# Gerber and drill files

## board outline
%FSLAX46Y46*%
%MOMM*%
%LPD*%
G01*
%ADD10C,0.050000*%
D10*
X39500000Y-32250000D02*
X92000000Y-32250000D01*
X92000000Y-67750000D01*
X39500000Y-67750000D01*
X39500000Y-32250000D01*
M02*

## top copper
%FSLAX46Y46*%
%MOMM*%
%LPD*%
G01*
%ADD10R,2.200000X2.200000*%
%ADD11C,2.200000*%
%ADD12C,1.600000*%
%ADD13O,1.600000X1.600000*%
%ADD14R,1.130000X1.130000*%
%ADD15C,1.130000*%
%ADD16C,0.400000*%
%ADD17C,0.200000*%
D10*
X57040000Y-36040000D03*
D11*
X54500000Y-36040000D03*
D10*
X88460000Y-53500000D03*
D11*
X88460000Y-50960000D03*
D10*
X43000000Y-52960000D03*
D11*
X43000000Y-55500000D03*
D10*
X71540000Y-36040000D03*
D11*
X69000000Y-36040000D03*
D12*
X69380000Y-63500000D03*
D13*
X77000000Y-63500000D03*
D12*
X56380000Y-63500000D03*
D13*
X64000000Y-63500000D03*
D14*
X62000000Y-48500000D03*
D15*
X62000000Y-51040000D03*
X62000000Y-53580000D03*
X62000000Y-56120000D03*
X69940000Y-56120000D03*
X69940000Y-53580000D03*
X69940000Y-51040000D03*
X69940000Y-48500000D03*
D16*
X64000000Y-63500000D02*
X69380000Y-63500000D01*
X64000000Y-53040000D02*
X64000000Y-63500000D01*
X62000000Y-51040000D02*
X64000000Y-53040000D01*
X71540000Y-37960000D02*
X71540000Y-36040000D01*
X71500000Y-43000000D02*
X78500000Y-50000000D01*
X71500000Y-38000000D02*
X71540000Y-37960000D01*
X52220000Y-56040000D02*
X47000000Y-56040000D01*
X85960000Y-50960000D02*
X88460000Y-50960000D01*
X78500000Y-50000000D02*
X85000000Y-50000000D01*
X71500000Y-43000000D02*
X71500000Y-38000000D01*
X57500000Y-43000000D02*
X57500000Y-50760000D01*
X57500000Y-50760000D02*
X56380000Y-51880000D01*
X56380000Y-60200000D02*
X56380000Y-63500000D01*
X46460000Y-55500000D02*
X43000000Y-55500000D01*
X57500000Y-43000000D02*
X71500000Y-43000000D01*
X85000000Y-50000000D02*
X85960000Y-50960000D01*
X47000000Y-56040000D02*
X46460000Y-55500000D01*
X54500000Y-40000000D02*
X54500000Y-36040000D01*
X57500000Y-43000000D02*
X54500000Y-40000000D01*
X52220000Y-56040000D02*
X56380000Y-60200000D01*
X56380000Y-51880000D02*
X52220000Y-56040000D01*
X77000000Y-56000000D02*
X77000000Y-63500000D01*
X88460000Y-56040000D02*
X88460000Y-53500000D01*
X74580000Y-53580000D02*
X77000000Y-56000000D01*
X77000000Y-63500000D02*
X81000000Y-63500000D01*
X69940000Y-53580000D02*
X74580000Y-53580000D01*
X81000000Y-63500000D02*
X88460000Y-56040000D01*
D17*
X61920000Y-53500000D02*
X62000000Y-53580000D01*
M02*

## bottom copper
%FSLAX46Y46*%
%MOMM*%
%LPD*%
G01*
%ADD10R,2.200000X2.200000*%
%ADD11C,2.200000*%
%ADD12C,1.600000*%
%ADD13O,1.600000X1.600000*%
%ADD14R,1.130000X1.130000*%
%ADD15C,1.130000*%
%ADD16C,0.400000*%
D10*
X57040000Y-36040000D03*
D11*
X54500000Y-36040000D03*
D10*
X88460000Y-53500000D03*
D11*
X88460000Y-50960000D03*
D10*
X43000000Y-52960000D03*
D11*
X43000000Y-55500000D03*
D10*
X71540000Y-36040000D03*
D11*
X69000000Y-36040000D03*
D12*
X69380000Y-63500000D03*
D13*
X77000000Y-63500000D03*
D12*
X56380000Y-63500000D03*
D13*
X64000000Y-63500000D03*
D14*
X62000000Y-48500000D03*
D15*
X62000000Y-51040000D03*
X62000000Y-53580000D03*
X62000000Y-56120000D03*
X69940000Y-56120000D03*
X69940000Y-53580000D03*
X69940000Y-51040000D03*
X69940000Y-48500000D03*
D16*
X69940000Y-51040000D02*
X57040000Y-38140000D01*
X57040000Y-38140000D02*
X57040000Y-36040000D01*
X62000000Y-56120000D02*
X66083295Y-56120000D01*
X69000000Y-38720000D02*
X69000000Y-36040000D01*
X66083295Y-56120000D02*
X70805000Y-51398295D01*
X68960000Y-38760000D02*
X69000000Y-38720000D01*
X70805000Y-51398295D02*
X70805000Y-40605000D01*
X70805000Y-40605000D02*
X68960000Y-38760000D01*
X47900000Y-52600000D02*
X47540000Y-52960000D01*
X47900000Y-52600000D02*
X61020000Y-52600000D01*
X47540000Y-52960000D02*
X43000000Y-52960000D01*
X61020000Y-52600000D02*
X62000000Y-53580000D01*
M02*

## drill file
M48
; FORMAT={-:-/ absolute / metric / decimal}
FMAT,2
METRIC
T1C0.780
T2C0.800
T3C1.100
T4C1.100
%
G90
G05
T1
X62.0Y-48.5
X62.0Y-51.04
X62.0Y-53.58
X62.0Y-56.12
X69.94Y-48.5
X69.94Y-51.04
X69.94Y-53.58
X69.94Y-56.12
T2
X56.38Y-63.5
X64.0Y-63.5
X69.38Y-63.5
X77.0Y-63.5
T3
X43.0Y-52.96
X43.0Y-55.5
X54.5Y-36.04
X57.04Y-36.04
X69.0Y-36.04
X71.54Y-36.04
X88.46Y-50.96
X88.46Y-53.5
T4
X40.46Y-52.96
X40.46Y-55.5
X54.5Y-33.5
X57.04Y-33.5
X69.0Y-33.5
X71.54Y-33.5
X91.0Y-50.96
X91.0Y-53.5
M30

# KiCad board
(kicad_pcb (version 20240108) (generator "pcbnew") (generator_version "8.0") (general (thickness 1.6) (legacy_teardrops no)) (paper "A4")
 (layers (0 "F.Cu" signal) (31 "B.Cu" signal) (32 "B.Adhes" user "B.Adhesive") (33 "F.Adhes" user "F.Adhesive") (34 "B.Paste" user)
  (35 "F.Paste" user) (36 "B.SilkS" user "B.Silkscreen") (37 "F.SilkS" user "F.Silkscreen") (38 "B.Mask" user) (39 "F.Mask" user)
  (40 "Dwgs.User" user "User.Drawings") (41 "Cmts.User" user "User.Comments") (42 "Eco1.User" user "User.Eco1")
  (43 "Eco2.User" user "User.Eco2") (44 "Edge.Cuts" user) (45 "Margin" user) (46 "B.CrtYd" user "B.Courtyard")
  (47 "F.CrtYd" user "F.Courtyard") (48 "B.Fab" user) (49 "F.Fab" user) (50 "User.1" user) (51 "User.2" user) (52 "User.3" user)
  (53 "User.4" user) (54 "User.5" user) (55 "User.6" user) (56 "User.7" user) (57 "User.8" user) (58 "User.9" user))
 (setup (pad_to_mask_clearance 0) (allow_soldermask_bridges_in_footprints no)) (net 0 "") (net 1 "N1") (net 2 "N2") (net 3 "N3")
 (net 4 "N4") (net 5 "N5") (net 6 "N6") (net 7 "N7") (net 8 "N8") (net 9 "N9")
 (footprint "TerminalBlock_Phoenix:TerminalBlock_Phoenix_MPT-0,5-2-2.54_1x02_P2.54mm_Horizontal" (layer "F.Cu") (at 57.04 36.04 180)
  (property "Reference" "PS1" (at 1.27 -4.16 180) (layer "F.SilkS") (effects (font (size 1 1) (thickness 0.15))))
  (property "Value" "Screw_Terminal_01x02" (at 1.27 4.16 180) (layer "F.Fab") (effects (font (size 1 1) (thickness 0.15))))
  (pad "" np_thru_hole circle (at 0 2.54 180) (size 1.1 1.1) (drill 1.1) (layers "*.Cu" "*.Mask"))
  (pad "" np_thru_hole circle (at 2.54 2.54 180) (size 1.1 1.1) (drill 1.1) (layers "*.Cu" "*.Mask"))
  (pad "1" thru_hole rect (at 0 0 180) (size 2.2 2.2) (drill 1.1) (layers "*.Cu" "*.Mask") (remove_unused_layers no) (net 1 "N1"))
  (pad "2" thru_hole circle (at 2.54 0 180) (size 2.2 2.2) (drill 1.1) (layers "*.Cu" "*.Mask") (remove_unused_layers no) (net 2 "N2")))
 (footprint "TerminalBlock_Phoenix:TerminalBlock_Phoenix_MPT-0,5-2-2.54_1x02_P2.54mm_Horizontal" (layer "F.Cu") (at 88.46 53.5 90)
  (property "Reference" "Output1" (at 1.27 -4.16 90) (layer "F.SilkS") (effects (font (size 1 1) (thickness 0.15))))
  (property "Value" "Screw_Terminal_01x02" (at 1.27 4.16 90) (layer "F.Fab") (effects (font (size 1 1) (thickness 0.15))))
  (pad "" np_thru_hole circle (at 0 2.54 90) (size 1.1 1.1) (drill 1.1) (layers "*.Cu" "*.Mask"))
  (pad "" np_thru_hole circle (at 2.54 2.54 90) (size 1.1 1.1) (drill 1.1) (layers "*.Cu" "*.Mask"))
  (pad "1" thru_hole rect (at 0 0 90) (size 2.2 2.2) (drill 1.1) (layers "*.Cu" "*.Mask") (remove_unused_layers no) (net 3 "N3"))
  (pad "2" thru_hole circle (at 2.54 0 90) (size 2.2 2.2) (drill 1.1) (layers "*.Cu" "*.Mask") (remove_unused_layers no) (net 2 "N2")))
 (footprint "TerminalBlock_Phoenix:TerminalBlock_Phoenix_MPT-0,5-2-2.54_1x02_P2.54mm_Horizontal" (layer "F.Cu") (at 43 52.96 -90)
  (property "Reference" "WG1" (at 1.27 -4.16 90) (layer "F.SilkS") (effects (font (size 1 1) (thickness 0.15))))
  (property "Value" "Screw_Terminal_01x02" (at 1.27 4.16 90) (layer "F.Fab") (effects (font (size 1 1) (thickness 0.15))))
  (pad "" np_thru_hole circle (at 0 2.54 270) (size 1.1 1.1) (drill 1.1) (layers "*.Cu" "*.Mask"))
  (pad "" np_thru_hole circle (at 2.54 2.54 270) (size 1.1 1.1) (drill 1.1) (layers "*.Cu" "*.Mask"))
  (pad "1" thru_hole rect (at 0 0 270) (size 2.2 2.2) (drill 1.1) (layers "*.Cu" "*.Mask") (remove_unused_layers no) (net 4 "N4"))
  (pad "2" thru_hole circle (at 2.54 0 270) (size 2.2 2.2) (drill 1.1) (layers "*.Cu" "*.Mask") (remove_unused_layers no) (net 2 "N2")))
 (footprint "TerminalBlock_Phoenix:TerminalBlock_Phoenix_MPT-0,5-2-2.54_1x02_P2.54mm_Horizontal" (layer "F.Cu") (at 71.54 36.04 180)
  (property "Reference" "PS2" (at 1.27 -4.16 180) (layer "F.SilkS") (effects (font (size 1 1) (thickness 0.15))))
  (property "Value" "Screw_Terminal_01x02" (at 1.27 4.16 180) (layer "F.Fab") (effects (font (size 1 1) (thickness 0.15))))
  (pad "" np_thru_hole circle (at 0 2.54 180) (size 1.1 1.1) (drill 1.1) (layers "*.Cu" "*.Mask"))
  (pad "" np_thru_hole circle (at 2.54 2.54 180) (size 1.1 1.1) (drill 1.1) (layers "*.Cu" "*.Mask"))
  (pad "1" thru_hole rect (at 0 0 180) (size 2.2 2.2) (drill 1.1) (layers "*.Cu" "*.Mask") (remove_unused_layers no) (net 2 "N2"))
  (pad "2" thru_hole circle (at 2.54 0 180) (size 2.2 2.2) (drill 1.1) (layers "*.Cu" "*.Mask") (remove_unused_layers no) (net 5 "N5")))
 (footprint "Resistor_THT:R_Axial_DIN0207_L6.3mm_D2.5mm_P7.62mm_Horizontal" (layer "F.Cu") (at 69.38 63.5)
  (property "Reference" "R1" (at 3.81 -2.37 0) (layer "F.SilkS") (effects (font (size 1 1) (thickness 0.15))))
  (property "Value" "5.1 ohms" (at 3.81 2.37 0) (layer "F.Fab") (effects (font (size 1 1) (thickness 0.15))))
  (pad "1" thru_hole circle (at 0 0) (size 1.6 1.6) (drill 0.8) (layers "*.Cu" "*.Mask") (remove_unused_layers no) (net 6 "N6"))
  (pad "2" thru_hole oval (at 7.62 0) (size 1.6 1.6) (drill 0.8) (layers "*.Cu" "*.Mask") (remove_unused_layers no) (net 3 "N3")))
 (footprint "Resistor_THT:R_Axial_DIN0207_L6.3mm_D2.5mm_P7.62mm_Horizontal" (layer "F.Cu") (at 56.38 63.5)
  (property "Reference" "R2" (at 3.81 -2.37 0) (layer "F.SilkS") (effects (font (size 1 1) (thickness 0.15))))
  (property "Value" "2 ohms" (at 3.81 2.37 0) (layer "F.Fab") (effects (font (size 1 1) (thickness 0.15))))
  (pad "1" thru_hole circle (at 0 0) (size 1.6 1.6) (drill 0.8) (layers "*.Cu" "*.Mask") (remove_unused_layers no) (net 2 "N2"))
  (pad "2" thru_hole oval (at 7.62 0) (size 1.6 1.6) (drill 0.8) (layers "*.Cu" "*.Mask") (remove_unused_layers no) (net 6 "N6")))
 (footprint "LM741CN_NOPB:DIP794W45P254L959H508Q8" (layer "F.Cu") (at 65.97 52.31)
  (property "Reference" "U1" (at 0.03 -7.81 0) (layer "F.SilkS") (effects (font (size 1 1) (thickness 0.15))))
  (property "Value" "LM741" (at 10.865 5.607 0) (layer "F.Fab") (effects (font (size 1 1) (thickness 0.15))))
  (pad "1" thru_hole rect (at -3.97 -3.81) (size 1.13 1.13) (drill 0.78) (layers "*.Cu" "*.Mask") (remove_unused_layers no) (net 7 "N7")
   (solder_mask_margin 0.102))
  (pad "2" thru_hole circle (at -3.97 -1.27) (size 1.13 1.13) (drill 0.78) (layers "*.Cu" "*.Mask") (remove_unused_layers no) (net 6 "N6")
   (solder_mask_margin 0.102))
  (pad "3" thru_hole circle (at -3.97 1.27) (size 1.13 1.13) (drill 0.78) (layers "*.Cu" "*.Mask") (remove_unused_layers no) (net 4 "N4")
   (solder_mask_margin 0.102))
  (pad "4" thru_hole circle (at -3.97 3.81) (size 1.13 1.13) (drill 0.78) (layers "*.Cu" "*.Mask") (remove_unused_layers no) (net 5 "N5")
   (solder_mask_margin 0.102))
  (pad "5" thru_hole circle (at 3.97 3.81) (size 1.13 1.13) (drill 0.78) (layers "*.Cu" "*.Mask") (remove_unused_layers no) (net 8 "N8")
   (solder_mask_margin 0.102))
  (pad "6" thru_hole circle (at 3.97 1.27) (size 1.13 1.13) (drill 0.78) (layers "*.Cu" "*.Mask") (remove_unused_layers no) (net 3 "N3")
   (solder_mask_margin 0.102))
  (pad "7" thru_hole circle (at 3.97 -1.27) (size 1.13 1.13) (drill 0.78) (layers "*.Cu" "*.Mask") (remove_unused_layers no) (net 1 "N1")
   (solder_mask_margin 0.102))
  (pad "8" thru_hole circle (at 3.97 -3.81) (size 1.13 1.13) (drill 0.78) (layers "*.Cu" "*.Mask") (remove_unused_layers no) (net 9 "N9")
   (solder_mask_margin 0.102)))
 (gr_rect (start 39.5 32.25) (end 92 67.75) (stroke (width 0.05) (type default)) (fill none) (layer "Edge.Cuts"))
 (segment (start 64 63.5) (end 69.38 63.5) (width 0.4) (layer "F.Cu") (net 6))
 (segment (start 64 53.04) (end 64 63.5) (width 0.4) (layer "F.Cu") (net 6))
 (segment (start 62 51.04) (end 64 53.04) (width 0.4) (layer "F.Cu") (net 6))
 (segment (start 71.54 37.96) (end 71.54 36.04) (width 0.4) (layer "F.Cu") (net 2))
 (segment (start 71.5 43) (end 78.5 50) (width 0.4) (layer "F.Cu") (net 2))
 (segment (start 71.5 38) (end 71.54 37.96) (width 0.4) (layer "F.Cu") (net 2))
 (segment (start 52.22 56.04) (end 47 56.04) (width 0.4) (layer "F.Cu") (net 2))
 (segment (start 85.96 50.96) (end 88.46 50.96) (width 0.4) (layer "F.Cu") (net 2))
 (segment (start 78.5 50) (end 85 50) (width 0.4) (layer "F.Cu") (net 2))
 (segment (start 71.5 43) (end 71.5 38) (width 0.4) (layer "F.Cu") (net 2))
 (segment (start 57.5 43) (end 57.5 50.76) (width 0.4) (layer "F.Cu") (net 2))
 (segment (start 57.5 50.76) (end 56.38 51.88) (width 0.4) (layer "F.Cu") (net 2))
 (segment (start 56.38 60.2) (end 56.38 63.5) (width 0.4) (layer "F.Cu") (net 2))
 (segment (start 46.46 55.5) (end 43 55.5) (width 0.4) (layer "F.Cu") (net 2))
 (segment (start 57.5 43) (end 71.5 43) (width 0.4) (layer "F.Cu") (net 2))
 (segment (start 85 50) (end 85.96 50.96) (width 0.4) (layer "F.Cu") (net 2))
 (segment (start 47 56.04) (end 46.46 55.5) (width 0.4) (layer "F.Cu") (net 2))
 (segment (start 54.5 40) (end 54.5 36.04) (width 0.4) (layer "F.Cu") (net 2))
 (segment (start 57.5 43) (end 54.5 40) (width 0.4) (layer "F.Cu") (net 2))
 (segment (start 52.22 56.04) (end 56.38 60.2) (width 0.4) (layer "F.Cu") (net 2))
 (segment (start 56.38 51.88) (end 52.22 56.04) (width 0.4) (layer "F.Cu") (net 2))
 (segment (start 77 56) (end 77 63.5) (width 0.4) (layer "F.Cu") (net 3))
 (segment (start 88.46 56.04) (end 88.46 53.5) (width 0.4) (layer "F.Cu") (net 3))
 (segment (start 74.58 53.58) (end 77 56) (width 0.4) (layer "F.Cu") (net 3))
 (segment (start 77 63.5) (end 81 63.5) (width 0.4) (layer "F.Cu") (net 3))
 (segment (start 69.94 53.58) (end 74.58 53.58) (width 0.4) (layer "F.Cu") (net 3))
 (segment (start 81 63.5) (end 88.46 56.04) (width 0.4) (layer "F.Cu") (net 3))
 (segment (start 69.94 51.04) (end 57.04 38.14) (width 0.4) (layer "B.Cu") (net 1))
 (segment (start 57.04 38.14) (end 57.04 36.04) (width 0.4) (layer "B.Cu") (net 1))
 (segment (start 62 56.12) (end 66.083295 56.12) (width 0.4) (layer "B.Cu") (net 5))
 (segment (start 69 38.72) (end 69 36.04) (width 0.4) (layer "B.Cu") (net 5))
 (segment (start 66.083295 56.12) (end 70.805 51.398295) (width 0.4) (layer "B.Cu") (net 5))
 (segment (start 68.96 38.76) (end 69 38.72) (width 0.4) (layer "B.Cu") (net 5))
 (segment (start 70.805 51.398295) (end 70.805 40.605) (width 0.4) (layer "B.Cu") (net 5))
 (segment (start 70.805 40.605) (end 68.96 38.76) (width 0.4) (layer "B.Cu") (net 5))
 (segment (start 61.92 53.5) (end 62 53.58) (width 0.2) (layer "F.Cu") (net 4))
 (segment (start 47.9 52.6) (end 47.54 52.96) (width 0.4) (layer "B.Cu") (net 4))
 (segment (start 47.9 52.6) (end 61.02 52.6) (width 0.4) (layer "B.Cu") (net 4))
 (segment (start 47.54 52.96) (end 43 52.96) (width 0.4) (layer "B.Cu") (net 4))
 (segment (start 61.02 52.6) (end 62 53.58) (width 0.4) (layer "B.Cu") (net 4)))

